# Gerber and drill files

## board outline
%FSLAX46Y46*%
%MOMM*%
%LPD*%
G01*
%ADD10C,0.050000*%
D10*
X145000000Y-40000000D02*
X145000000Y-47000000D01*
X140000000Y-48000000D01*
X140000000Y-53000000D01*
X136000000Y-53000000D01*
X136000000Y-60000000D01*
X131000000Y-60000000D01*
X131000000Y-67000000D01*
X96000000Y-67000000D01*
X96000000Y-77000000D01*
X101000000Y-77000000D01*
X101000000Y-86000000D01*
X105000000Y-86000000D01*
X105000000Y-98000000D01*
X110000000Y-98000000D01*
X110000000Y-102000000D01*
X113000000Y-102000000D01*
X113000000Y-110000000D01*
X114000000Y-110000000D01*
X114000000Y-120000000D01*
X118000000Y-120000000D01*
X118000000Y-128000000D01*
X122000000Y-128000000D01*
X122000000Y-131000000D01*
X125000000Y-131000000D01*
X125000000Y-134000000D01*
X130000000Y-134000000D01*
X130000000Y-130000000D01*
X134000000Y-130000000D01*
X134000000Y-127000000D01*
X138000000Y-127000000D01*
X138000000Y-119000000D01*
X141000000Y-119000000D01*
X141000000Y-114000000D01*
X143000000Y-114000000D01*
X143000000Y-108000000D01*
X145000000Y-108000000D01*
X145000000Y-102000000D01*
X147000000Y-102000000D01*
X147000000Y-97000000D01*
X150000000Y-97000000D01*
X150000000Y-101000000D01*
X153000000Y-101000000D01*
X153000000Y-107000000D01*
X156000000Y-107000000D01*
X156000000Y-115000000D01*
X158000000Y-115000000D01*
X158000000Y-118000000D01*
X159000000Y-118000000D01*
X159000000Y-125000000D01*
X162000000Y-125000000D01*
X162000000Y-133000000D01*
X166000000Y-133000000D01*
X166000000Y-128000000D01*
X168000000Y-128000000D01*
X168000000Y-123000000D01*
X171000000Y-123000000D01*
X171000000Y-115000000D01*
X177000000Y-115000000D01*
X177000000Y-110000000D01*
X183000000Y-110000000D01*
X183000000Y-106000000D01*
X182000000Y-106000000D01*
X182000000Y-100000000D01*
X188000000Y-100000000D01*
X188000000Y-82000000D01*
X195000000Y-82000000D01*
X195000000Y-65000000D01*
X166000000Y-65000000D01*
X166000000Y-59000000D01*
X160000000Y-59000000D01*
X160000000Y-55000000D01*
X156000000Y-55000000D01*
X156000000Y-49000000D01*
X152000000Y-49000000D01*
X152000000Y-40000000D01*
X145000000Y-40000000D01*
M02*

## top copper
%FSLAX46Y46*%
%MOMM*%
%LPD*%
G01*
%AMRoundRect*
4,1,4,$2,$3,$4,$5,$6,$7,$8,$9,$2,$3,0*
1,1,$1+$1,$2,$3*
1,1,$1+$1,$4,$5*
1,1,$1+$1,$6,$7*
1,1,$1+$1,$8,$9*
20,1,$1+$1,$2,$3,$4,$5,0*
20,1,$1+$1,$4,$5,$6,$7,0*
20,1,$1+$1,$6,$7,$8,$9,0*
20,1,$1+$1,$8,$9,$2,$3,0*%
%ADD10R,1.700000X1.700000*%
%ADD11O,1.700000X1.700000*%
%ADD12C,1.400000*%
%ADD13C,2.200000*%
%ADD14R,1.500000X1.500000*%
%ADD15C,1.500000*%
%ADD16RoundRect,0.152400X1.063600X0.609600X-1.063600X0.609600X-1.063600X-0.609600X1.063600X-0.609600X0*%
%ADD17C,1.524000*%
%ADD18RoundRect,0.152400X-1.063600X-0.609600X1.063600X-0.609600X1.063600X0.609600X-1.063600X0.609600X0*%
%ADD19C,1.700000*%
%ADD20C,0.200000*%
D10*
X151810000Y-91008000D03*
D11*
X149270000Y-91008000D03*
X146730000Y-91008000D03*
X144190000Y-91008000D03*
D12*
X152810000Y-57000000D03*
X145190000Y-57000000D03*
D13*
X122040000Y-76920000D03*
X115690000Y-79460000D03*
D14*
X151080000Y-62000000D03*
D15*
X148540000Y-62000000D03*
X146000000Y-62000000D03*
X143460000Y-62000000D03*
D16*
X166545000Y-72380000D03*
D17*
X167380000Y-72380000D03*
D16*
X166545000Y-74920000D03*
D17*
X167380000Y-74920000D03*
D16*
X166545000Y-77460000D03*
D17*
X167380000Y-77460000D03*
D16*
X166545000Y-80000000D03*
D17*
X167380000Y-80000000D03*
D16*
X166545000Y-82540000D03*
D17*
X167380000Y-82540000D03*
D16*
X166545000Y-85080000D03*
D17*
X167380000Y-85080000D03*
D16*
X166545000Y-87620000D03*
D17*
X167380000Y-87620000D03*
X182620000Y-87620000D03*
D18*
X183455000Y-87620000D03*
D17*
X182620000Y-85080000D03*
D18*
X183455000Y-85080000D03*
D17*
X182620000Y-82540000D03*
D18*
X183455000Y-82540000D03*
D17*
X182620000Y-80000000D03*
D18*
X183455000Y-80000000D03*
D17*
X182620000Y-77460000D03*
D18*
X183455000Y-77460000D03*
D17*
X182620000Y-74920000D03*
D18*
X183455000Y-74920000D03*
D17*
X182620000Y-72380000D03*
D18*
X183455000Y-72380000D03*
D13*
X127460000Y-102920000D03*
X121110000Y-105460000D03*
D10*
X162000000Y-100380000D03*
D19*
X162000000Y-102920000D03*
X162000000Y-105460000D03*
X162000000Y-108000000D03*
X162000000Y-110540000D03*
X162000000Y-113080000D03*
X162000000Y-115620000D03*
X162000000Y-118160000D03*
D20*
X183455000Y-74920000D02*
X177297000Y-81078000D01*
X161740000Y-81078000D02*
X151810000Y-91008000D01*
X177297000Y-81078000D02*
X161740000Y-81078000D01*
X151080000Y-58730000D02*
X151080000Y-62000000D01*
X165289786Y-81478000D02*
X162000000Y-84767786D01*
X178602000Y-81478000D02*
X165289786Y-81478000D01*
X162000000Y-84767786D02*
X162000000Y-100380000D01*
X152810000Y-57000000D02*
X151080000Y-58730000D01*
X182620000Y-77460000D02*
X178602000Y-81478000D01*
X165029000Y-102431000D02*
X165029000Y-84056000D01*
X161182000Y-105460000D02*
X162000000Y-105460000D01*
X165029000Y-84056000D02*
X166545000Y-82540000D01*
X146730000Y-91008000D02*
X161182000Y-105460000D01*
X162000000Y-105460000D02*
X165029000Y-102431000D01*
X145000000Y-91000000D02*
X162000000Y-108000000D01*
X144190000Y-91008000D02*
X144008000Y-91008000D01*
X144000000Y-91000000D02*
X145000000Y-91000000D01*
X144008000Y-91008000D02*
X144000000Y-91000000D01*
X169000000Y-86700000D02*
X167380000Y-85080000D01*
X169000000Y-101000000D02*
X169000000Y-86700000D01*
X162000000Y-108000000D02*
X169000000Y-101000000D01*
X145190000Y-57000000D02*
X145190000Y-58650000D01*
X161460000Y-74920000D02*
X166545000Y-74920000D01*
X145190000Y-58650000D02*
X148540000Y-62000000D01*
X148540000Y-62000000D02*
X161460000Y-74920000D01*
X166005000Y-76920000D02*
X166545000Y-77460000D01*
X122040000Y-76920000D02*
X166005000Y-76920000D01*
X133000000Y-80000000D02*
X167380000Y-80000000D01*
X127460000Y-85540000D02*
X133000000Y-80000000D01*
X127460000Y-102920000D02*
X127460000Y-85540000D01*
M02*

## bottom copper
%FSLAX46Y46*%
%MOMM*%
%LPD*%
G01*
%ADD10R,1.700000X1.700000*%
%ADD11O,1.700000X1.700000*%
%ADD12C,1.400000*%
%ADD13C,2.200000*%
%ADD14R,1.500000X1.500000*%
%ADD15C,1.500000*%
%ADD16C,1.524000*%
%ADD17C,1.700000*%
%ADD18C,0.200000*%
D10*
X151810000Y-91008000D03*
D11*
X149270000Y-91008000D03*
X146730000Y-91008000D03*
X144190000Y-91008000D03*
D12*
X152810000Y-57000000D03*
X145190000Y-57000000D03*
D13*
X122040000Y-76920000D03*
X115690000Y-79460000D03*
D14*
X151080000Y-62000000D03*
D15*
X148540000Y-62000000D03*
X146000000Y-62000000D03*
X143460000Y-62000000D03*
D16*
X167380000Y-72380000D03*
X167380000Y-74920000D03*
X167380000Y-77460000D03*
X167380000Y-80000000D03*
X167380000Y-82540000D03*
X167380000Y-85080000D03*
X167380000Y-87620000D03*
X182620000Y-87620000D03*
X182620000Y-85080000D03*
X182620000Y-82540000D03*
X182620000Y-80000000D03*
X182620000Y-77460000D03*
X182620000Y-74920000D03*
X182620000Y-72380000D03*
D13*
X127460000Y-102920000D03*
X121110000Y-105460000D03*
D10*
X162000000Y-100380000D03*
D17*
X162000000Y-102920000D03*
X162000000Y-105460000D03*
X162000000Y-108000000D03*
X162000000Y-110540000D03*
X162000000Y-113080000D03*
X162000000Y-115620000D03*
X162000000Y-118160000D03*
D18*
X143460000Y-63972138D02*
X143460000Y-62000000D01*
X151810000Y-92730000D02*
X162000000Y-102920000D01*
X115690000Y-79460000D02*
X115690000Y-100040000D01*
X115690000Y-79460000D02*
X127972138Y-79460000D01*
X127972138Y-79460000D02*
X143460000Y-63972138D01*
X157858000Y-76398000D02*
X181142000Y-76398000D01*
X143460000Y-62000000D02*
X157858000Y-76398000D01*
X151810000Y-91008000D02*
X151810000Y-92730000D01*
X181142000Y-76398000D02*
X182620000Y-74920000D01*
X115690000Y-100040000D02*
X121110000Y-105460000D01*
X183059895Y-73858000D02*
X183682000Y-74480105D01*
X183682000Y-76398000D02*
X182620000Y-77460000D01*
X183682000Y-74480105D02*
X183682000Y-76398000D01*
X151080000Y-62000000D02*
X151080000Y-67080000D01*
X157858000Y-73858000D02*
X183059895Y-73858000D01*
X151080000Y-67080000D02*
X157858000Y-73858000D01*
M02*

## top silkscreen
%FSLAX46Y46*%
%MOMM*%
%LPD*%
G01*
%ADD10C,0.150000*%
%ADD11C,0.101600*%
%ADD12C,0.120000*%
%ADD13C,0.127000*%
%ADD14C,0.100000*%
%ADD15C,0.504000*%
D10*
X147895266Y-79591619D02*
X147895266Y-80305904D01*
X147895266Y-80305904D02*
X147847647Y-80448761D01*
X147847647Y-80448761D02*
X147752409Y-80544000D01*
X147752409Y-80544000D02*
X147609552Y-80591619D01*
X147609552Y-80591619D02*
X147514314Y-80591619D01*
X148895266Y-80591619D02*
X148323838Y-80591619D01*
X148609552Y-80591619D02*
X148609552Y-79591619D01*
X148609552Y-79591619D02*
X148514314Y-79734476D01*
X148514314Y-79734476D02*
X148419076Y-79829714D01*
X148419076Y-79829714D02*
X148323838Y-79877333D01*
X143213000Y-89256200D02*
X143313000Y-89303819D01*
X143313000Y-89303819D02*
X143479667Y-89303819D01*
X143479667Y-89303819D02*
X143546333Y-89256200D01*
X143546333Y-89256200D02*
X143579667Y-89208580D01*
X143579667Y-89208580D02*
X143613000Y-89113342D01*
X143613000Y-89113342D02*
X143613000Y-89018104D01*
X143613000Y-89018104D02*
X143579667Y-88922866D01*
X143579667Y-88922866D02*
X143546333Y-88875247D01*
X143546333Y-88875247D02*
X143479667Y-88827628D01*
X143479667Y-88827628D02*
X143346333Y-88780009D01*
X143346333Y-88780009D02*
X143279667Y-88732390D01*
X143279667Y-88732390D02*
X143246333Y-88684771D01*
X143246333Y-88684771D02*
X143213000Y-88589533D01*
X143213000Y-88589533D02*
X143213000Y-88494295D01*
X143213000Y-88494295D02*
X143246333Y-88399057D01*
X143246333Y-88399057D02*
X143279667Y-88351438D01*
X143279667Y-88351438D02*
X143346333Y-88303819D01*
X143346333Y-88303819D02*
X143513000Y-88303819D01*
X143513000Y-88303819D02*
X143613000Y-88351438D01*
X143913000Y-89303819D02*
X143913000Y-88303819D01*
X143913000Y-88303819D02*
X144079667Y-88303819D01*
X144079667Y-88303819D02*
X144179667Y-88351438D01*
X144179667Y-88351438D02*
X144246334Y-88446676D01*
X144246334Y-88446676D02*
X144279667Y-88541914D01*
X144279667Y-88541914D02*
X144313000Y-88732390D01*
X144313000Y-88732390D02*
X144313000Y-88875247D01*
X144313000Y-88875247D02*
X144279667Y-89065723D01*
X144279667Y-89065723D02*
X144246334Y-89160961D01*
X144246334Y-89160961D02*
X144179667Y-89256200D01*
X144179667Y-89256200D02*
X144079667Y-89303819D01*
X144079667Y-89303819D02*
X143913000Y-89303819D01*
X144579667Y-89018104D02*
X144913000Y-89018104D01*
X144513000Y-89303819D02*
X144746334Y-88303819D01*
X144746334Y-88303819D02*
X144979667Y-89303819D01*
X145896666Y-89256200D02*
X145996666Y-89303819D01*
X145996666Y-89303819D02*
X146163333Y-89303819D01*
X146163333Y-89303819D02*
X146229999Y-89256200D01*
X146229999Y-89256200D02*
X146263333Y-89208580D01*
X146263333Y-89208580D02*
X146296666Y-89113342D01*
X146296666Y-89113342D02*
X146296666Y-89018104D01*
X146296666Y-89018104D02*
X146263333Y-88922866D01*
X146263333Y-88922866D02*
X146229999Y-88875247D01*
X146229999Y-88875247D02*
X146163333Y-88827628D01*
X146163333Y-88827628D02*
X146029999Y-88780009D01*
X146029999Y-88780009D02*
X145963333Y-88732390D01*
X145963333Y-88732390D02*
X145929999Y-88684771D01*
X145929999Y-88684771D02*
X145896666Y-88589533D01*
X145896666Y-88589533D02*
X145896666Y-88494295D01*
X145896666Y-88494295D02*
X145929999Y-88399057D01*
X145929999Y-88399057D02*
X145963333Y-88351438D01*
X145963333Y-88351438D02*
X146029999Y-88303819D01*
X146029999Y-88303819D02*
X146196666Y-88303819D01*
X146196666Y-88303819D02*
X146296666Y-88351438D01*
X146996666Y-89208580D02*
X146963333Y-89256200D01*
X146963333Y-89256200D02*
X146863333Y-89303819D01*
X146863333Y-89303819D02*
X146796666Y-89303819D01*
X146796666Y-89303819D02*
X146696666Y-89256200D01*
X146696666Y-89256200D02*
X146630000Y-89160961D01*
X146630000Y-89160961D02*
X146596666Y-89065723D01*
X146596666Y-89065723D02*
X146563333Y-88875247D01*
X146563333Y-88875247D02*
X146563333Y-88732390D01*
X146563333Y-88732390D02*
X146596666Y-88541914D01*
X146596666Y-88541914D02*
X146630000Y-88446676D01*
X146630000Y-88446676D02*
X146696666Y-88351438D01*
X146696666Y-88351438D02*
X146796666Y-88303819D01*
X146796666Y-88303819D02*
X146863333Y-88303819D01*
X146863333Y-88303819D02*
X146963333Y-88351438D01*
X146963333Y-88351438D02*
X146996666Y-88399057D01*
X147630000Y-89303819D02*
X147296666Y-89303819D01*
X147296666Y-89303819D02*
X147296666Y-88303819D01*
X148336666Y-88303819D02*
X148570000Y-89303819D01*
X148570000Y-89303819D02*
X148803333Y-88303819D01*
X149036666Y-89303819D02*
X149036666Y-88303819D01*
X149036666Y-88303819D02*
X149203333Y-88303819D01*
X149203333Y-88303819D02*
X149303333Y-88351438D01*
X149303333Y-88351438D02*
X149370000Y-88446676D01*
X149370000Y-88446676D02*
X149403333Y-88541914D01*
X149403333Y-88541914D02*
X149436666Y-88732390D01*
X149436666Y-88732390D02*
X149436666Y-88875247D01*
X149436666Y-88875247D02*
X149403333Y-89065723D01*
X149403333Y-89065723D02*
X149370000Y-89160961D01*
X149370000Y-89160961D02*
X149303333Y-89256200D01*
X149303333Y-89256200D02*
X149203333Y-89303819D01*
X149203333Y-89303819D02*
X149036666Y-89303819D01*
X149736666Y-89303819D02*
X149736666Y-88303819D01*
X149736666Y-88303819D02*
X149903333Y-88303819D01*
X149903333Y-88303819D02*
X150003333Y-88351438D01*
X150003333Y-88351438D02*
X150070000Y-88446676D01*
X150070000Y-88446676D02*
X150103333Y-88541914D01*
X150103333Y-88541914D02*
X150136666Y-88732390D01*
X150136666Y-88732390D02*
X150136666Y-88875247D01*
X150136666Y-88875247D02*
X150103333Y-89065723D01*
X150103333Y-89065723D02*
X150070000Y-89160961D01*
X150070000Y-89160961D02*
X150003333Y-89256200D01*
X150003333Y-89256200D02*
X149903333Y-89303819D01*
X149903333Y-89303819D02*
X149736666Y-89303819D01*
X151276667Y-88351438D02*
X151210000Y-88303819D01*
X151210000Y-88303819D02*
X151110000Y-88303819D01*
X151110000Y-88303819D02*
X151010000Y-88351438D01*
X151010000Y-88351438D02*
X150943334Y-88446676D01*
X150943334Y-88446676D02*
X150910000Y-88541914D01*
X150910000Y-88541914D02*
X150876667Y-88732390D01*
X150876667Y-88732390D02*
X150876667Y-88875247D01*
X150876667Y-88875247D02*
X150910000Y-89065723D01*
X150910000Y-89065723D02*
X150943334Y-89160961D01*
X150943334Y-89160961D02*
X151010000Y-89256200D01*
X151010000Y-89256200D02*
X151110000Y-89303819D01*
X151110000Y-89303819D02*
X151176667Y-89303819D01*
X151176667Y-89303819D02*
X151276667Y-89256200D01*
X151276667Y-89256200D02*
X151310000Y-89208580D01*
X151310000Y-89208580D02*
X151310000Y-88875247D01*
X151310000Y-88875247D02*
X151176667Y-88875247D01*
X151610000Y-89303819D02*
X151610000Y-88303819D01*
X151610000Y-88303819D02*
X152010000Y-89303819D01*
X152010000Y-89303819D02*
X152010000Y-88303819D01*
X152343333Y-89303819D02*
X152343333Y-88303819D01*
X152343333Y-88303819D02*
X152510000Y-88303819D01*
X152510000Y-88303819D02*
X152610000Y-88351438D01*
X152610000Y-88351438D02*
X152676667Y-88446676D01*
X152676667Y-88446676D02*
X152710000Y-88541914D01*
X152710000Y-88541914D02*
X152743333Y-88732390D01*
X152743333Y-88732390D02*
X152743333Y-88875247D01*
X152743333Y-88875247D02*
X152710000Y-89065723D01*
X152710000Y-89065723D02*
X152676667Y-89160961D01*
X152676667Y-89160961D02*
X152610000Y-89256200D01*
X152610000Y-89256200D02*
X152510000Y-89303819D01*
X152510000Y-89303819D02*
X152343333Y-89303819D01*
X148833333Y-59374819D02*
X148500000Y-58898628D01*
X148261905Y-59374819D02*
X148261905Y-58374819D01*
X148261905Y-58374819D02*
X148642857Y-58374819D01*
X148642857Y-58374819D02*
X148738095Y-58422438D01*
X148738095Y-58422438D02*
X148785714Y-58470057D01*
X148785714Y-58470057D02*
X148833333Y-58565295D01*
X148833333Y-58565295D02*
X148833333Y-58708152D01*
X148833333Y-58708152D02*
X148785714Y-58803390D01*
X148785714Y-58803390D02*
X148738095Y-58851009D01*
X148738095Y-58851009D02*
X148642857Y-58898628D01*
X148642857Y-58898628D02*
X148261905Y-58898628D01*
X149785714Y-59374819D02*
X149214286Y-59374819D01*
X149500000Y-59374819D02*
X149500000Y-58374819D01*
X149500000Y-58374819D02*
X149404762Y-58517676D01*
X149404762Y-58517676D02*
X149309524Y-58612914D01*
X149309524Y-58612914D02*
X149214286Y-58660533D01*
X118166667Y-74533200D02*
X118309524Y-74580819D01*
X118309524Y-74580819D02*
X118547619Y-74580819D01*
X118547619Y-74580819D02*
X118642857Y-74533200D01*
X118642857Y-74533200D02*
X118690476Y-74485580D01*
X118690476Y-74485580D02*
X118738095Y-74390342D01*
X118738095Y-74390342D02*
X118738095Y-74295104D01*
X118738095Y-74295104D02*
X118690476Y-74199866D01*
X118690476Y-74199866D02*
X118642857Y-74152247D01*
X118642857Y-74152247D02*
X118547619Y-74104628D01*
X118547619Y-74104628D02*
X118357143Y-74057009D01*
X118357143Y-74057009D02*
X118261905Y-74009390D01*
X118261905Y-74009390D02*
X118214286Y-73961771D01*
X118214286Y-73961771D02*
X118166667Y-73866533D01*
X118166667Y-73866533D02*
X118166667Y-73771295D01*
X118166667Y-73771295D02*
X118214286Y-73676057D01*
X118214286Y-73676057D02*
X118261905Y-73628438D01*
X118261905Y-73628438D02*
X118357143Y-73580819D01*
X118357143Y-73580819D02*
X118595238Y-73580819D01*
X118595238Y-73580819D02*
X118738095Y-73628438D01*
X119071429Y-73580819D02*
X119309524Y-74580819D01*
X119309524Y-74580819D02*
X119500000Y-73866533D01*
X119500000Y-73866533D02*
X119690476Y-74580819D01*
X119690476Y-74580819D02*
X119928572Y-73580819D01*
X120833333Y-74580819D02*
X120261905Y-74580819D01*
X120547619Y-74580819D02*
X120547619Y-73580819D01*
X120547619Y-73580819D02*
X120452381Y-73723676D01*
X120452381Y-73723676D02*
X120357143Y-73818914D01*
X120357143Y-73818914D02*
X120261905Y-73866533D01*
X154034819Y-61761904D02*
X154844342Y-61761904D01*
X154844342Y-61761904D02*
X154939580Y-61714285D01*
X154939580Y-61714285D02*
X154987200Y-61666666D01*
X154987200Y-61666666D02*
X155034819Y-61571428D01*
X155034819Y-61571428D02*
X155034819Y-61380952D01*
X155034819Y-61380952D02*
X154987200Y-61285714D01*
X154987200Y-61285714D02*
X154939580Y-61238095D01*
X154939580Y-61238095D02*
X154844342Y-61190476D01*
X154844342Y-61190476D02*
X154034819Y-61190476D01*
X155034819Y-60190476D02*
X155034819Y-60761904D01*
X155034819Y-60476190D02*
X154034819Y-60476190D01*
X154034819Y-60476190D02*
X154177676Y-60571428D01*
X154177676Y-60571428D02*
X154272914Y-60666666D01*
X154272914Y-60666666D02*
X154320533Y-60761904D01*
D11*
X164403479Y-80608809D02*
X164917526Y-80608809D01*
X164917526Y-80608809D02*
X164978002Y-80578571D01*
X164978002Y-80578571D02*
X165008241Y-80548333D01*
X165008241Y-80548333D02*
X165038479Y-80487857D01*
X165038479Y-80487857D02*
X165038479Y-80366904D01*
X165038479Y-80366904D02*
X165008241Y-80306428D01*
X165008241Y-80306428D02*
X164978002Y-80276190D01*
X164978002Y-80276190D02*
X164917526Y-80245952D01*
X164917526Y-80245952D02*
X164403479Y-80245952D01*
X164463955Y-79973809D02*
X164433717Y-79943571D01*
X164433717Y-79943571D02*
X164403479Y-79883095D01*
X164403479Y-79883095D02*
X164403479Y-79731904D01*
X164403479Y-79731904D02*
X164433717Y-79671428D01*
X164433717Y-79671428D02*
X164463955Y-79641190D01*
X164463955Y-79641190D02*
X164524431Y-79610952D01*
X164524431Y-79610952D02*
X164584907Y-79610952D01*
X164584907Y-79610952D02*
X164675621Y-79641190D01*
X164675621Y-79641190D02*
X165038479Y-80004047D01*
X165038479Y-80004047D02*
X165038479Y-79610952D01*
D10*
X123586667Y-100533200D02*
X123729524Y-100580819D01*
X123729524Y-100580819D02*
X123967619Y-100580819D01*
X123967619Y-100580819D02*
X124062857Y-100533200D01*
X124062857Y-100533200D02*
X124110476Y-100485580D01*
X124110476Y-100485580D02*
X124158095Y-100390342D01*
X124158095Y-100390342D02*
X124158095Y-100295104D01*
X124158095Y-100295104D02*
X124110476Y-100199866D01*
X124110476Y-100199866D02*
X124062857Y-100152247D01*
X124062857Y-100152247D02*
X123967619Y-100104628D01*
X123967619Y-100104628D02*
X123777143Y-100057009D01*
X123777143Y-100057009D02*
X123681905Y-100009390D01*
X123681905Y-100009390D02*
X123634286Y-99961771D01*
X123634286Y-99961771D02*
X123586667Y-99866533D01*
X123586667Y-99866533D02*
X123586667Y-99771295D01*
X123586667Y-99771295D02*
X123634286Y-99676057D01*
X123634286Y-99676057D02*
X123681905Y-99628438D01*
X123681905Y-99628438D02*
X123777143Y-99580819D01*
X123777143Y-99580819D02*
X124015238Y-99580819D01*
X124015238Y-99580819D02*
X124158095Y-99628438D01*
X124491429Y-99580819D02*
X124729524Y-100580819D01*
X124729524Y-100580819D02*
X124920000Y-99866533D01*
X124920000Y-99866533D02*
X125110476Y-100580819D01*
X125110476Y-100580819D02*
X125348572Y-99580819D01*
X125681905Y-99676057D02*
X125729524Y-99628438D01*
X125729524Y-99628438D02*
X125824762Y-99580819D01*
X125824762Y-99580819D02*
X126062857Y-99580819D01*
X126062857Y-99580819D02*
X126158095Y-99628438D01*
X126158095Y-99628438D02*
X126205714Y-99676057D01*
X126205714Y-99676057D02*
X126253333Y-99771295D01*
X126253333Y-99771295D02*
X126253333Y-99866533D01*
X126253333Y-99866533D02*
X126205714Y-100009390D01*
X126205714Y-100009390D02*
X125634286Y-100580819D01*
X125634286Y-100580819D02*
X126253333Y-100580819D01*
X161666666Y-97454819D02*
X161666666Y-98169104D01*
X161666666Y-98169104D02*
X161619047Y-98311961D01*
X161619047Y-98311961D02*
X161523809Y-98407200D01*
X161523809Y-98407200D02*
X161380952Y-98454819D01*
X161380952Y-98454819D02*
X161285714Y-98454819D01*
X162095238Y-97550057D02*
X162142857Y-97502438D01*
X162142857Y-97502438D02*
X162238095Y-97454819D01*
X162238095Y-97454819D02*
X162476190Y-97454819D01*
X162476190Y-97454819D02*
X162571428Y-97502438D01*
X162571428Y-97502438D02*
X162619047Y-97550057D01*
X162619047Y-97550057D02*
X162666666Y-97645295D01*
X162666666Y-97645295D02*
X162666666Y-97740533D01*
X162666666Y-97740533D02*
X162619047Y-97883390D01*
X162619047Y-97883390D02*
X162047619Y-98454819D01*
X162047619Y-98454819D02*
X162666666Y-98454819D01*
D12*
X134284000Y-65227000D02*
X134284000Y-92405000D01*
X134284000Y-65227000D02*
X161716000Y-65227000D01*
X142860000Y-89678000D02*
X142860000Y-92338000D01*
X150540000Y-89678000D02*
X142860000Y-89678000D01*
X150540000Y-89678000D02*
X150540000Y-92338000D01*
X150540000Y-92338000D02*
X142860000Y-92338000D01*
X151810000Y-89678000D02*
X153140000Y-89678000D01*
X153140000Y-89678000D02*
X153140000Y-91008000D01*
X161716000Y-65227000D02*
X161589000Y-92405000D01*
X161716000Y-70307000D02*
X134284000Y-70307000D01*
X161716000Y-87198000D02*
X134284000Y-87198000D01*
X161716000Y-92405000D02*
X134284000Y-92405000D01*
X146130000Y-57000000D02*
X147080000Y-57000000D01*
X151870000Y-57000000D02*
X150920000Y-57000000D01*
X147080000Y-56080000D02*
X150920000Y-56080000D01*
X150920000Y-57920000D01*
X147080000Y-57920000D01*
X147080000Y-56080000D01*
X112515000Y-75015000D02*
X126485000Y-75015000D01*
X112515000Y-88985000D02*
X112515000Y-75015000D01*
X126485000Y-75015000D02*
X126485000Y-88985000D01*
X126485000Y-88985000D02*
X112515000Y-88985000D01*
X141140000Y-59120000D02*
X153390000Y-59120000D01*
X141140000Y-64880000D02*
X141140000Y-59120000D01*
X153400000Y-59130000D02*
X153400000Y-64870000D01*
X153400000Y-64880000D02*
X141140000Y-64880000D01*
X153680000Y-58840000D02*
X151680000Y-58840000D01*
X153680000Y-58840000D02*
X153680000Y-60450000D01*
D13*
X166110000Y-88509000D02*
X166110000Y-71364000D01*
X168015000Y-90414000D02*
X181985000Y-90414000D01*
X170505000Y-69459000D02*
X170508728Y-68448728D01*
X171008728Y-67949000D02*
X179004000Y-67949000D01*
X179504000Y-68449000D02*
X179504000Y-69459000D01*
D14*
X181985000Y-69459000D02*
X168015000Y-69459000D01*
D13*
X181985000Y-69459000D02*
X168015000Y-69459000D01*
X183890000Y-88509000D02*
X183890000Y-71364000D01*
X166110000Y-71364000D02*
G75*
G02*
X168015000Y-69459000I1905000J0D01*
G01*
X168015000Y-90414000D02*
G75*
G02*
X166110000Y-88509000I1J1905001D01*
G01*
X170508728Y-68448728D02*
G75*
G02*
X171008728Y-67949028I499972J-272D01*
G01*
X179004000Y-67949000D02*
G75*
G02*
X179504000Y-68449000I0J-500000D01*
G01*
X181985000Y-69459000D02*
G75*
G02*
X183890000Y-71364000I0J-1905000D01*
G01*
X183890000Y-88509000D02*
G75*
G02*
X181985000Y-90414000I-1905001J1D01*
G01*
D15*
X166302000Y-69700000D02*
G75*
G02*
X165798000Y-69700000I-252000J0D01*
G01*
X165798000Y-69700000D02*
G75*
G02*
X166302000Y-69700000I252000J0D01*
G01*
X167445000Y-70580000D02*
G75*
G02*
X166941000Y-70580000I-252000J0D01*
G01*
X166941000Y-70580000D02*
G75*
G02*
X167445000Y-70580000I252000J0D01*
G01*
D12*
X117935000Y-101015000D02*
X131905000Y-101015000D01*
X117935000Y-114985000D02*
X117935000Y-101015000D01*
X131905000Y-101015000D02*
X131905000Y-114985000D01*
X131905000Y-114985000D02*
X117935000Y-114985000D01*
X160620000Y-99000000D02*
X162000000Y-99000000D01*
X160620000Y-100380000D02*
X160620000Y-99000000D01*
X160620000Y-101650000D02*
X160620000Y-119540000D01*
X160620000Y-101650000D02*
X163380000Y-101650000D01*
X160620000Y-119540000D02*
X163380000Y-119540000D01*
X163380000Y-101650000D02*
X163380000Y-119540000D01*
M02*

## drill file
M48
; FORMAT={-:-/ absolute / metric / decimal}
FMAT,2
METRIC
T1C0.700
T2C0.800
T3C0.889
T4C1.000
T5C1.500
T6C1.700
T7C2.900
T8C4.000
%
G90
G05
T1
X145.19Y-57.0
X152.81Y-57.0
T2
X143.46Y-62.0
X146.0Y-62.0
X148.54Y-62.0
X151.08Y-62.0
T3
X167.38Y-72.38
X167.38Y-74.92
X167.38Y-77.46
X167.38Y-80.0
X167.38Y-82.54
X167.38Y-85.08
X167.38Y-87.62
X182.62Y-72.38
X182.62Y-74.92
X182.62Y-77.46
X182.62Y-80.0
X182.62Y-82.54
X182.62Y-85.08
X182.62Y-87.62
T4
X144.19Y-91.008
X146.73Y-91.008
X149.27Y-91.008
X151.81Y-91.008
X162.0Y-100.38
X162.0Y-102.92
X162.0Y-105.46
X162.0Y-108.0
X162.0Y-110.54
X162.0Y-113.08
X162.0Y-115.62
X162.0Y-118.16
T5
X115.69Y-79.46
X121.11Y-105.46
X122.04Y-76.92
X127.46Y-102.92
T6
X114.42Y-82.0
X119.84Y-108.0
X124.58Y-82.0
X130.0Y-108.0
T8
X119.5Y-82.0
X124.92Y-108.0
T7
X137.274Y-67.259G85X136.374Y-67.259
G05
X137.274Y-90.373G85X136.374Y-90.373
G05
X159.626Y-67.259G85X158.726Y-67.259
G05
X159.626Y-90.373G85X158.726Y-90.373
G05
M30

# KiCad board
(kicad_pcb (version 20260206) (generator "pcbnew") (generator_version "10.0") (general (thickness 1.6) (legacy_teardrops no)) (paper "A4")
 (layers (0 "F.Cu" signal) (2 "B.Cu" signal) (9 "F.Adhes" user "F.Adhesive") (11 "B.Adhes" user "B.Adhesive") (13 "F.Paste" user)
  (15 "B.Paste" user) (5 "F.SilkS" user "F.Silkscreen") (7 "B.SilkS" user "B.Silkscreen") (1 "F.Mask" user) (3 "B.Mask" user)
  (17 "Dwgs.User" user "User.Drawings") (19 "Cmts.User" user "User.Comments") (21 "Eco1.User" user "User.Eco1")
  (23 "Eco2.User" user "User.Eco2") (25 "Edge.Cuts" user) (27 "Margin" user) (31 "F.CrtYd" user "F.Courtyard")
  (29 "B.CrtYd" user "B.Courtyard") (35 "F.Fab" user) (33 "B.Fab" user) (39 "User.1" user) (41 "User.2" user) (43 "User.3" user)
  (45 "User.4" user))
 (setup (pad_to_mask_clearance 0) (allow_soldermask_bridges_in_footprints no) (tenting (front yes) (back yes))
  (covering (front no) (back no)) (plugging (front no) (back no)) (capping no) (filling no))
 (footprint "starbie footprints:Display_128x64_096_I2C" (layer "F.Cu") (at 148 91.008 180)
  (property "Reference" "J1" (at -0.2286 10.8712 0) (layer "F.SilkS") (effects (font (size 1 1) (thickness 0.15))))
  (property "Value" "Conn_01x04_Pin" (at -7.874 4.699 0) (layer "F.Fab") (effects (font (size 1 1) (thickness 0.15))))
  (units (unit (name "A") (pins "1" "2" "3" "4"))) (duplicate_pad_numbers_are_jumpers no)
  (fp_line (start 13.716 25.781) (end 13.716 -1.397) (stroke (width 0.12) (type solid)) (layer "F.SilkS"))
  (fp_line (start 13.716 25.781) (end -13.716 25.781) (stroke (width 0.12) (type solid)) (layer "F.SilkS"))
  (fp_line (start 5.14 1.33) (end 5.14 -1.33) (stroke (width 0.12) (type solid)) (layer "F.SilkS"))
  (fp_line (start -2.54 1.33) (end 5.14 1.33) (stroke (width 0.12) (type solid)) (layer "F.SilkS"))
  (fp_line (start -2.54 1.33) (end -2.54 -1.33) (stroke (width 0.12) (type solid)) (layer "F.SilkS"))
  (fp_line (start -2.54 -1.33) (end 5.14 -1.33) (stroke (width 0.12) (type solid)) (layer "F.SilkS"))
  (fp_line (start -3.81 1.33) (end -5.14 1.33) (stroke (width 0.12) (type solid)) (layer "F.SilkS"))
  (fp_line (start -5.14 1.33) (end -5.14 0) (stroke (width 0.12) (type solid)) (layer "F.SilkS"))
  (fp_line (start -13.716 25.781) (end -13.589 -1.397) (stroke (width 0.12) (type solid)) (layer "F.SilkS"))
  (fp_line (start -13.716 20.701) (end 13.716 20.701) (stroke (width 0.12) (type solid)) (layer "F.SilkS"))
  (fp_line (start -13.716 3.81) (end 13.716 3.81) (stroke (width 0.12) (type solid)) (layer "F.SilkS"))
  (fp_line (start -13.716 -1.397) (end 13.716 -1.397) (stroke (width 0.12) (type solid)) (layer "F.SilkS"))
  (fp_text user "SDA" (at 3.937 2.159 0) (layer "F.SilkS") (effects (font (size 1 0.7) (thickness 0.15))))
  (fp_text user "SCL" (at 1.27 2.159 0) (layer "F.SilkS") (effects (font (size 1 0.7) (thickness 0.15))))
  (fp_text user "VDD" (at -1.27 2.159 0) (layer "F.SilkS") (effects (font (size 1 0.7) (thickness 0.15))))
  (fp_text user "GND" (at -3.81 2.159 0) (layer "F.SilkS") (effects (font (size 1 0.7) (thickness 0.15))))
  (pad "" np_thru_hole oval (at -11.176 0.635 180) (size 3.8 2.9) (drill oval 3.8 2.9) (layers "*.Cu" "*.Mask"))
  (pad "" np_thru_hole oval (at -11.176 23.749 180) (size 3.8 2.9) (drill oval 3.8 2.9) (layers "*.Cu" "*.Mask"))
  (pad "" np_thru_hole oval (at 11.176 0.635 180) (size 3.8 2.9) (drill oval 3.8 2.9) (layers "*.Cu" "*.Mask"))
  (pad "" np_thru_hole oval (at 11.176 23.749 180) (size 3.8 2.9) (drill oval 3.8 2.9) (layers "*.Cu" "*.Mask"))
  (pad "1" thru_hole rect (at -3.81 0 270) (size 1.7 1.7) (drill 1) (layers "*.Cu" "*.Mask") (remove_unused_layers no) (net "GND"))
  (pad "2" thru_hole oval (at -1.27 0 270) (size 1.7 1.7) (drill 1) (layers "*.Cu" "*.Mask") (remove_unused_layers no) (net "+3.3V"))
  (pad "3" thru_hole oval (at 1.27 0 270) (size 1.7 1.7) (drill 1) (layers "*.Cu" "*.Mask") (remove_unused_layers no) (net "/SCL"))
  (pad "4" thru_hole oval (at 3.81 0 270) (size 1.7 1.7) (drill 1) (layers "*.Cu" "*.Mask") (remove_unused_layers no) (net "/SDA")))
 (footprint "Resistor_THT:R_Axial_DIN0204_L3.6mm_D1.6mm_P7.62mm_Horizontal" (layer "F.Cu") (at 152.81 57 180)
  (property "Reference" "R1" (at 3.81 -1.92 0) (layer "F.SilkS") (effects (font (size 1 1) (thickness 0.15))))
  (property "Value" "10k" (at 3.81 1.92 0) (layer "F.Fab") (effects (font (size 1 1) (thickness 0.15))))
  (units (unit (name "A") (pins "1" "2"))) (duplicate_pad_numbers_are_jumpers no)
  (fp_line (start 6.68 0) (end 5.73 0) (stroke (width 0.12) (type solid)) (layer "F.SilkS"))
  (fp_line (start 0.94 0) (end 1.89 0) (stroke (width 0.12) (type solid)) (layer "F.SilkS"))
  (fp_rect (start 1.89 -0.92) (end 5.73 0.92) (stroke (width 0.12) (type solid)) (fill no) (layer "F.SilkS"))
  (pad "1" thru_hole circle (at 0 0 180) (size 1.4 1.4) (drill 0.7) (layers "*.Cu" "*.Mask") (remove_unused_layers no) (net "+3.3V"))
  (pad "2" thru_hole circle (at 7.62 0 180) (size 1.4 1.4) (drill 0.7) (layers "*.Cu" "*.Mask") (remove_unused_layers no)
   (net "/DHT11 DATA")))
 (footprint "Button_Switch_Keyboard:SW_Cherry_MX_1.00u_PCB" (layer "F.Cu") (at 122.04 76.92)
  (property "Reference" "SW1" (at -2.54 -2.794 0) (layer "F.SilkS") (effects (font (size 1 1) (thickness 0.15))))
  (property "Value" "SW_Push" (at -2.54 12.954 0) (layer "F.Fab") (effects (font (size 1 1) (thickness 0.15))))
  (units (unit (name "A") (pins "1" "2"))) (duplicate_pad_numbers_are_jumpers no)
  (fp_line (start -9.525 -1.905) (end 4.445 -1.905) (stroke (width 0.12) (type solid)) (layer "F.SilkS"))
  (fp_line (start -9.525 12.065) (end -9.525 -1.905) (stroke (width 0.12) (type solid)) (layer "F.SilkS"))
  (fp_line (start 4.445 -1.905) (end 4.445 12.065) (stroke (width 0.12) (type solid)) (layer "F.SilkS"))
  (fp_line (start 4.445 12.065) (end -9.525 12.065) (stroke (width 0.12) (type solid)) (layer "F.SilkS"))
  (pad "" np_thru_hole circle (at -7.62 5.08) (size 1.7 1.7) (drill 1.7) (layers "*.Cu" "*.Mask"))
  (pad "" np_thru_hole circle (at -2.54 5.08) (size 4 4) (drill 4) (layers "*.Cu" "*.Mask"))
  (pad "" np_thru_hole circle (at 2.54 5.08) (size 1.7 1.7) (drill 1.7) (layers "*.Cu" "*.Mask"))
  (pad "1" thru_hole circle (at 0 0) (size 2.2 2.2) (drill 1.5) (layers "*.Cu" "*.Mask") (remove_unused_layers no) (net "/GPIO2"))
  (pad "2" thru_hole circle (at -6.35 2.54) (size 2.2 2.2) (drill 1.5) (layers "*.Cu" "*.Mask") (remove_unused_layers no) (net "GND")))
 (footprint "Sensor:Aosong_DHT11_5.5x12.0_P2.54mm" (layer "F.Cu") (at 151.08 62 -90)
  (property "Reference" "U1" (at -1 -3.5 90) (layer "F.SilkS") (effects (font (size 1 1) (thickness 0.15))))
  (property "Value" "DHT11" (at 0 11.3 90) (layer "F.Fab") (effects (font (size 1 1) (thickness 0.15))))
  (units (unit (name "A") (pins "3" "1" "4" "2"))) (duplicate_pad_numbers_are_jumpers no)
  (fp_line (start -2.88 9.94) (end -2.88 -2.31) (stroke (width 0.12) (type solid)) (layer "F.SilkS"))
  (fp_line (start 2.88 9.94) (end -2.88 9.94) (stroke (width 0.12) (type solid)) (layer "F.SilkS"))
  (fp_line (start -2.87 -2.32) (end 2.87 -2.32) (stroke (width 0.12) (type solid)) (layer "F.SilkS"))
  (fp_line (start 2.88 -2.32) (end 2.88 9.94) (stroke (width 0.12) (type solid)) (layer "F.SilkS"))
  (fp_line (start -3.16 -2.6) (end -3.16 -0.6) (stroke (width 0.12) (type solid)) (layer "F.SilkS"))
  (fp_line (start -3.16 -2.6) (end -1.55 -2.6) (stroke (width 0.12) (type solid)) (layer "F.SilkS"))
  (pad "1" thru_hole rect (at 0 0 270) (size 1.5 1.5) (drill 0.8) (layers "*.Cu" "*.Mask") (remove_unused_layers no) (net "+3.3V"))
  (pad "2" thru_hole circle (at 0 2.54 270) (size 1.5 1.5) (drill 0.8) (layers "*.Cu" "*.Mask") (remove_unused_layers no)
   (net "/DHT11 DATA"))
  (pad "3" thru_hole circle (at 0 5.08 270) (size 1.5 1.5) (drill 0.8) (layers "*.Cu" "*.Mask") (remove_unused_layers no)
   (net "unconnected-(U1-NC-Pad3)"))
  (pad "4" thru_hole circle (at 0 7.62 270) (size 1.5 1.5) (drill 0.8) (layers "*.Cu" "*.Mask") (remove_unused_layers no) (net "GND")))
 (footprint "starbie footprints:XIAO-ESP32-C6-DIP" (layer "F.Cu") (at 175 80 90)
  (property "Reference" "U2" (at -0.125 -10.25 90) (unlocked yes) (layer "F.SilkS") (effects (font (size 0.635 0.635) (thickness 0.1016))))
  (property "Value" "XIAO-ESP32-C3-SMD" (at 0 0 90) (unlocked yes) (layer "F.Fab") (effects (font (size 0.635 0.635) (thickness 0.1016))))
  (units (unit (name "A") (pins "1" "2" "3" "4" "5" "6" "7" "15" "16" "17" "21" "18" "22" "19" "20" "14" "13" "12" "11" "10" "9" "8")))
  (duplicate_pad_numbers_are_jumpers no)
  (fp_line (start -8.509 -8.89) (end 8.636 -8.89) (stroke (width 0.127) (type solid)) (layer "F.SilkS"))
  (fp_line (start -10.414 -6.985) (end -10.414 6.985) (stroke (width 0.127) (type solid)) (layer "F.SilkS"))
  (fp_line (start 10.541 -4.495) (end 11.551272 -4.491272) (stroke (width 0.127) (type solid)) (layer "F.SilkS"))
  (fp_line (start 12.051 -3.991272) (end 12.051 4.004) (stroke (width 0.127) (type solid)) (layer "F.SilkS"))
  (fp_line (start 11.551 4.504) (end 10.541 4.504) (stroke (width 0.127) (type solid)) (layer "F.SilkS"))
  (fp_line (start 10.541 6.985) (end 10.541 -6.985) (stroke (width 0.1) (type solid)) (layer "F.SilkS"))
  (fp_line (start 10.541 6.985) (end 10.541 -6.985) (stroke (width 0.127) (type solid)) (layer "F.SilkS"))
  (fp_line (start -8.509 8.89) (end 8.636 8.89) (stroke (width 0.127) (type solid)) (layer "F.SilkS"))
  (fp_arc (start 8.636 -8.89) (mid 9.983038 -8.332038) (end 10.541 -6.985) (stroke (width 0.127) (type solid)) (layer "F.SilkS"))
  (fp_arc (start -10.414 -6.985) (mid -9.856038 -8.332038) (end -8.509 -8.89) (stroke (width 0.127) (type solid)) (layer "F.SilkS"))
  (fp_arc (start 11.551272 -4.491272) (mid 11.904644 -4.344724) (end 12.051 -3.991272) (stroke (width 0.127) (type default))
   (layer "F.SilkS"))
  (fp_arc (start 12.051 4.004) (mid 11.904553 4.357553) (end 11.551 4.504) (stroke (width 0.127) (type default)) (layer "F.SilkS"))
  (fp_arc (start 10.541 6.985) (mid 9.983038 8.332038) (end 8.636 8.89) (stroke (width 0.127) (type solid)) (layer "F.SilkS"))
  (fp_arc (start -8.509 8.89) (mid -9.856038 8.332038) (end -10.414 6.985) (stroke (width 0.127) (type solid)) (layer "F.SilkS"))
  (fp_circle (center 10.3 -8.95) (end 10.554 -8.95) (stroke (width 0.5) (type solid)) (fill yes) (layer "F.SilkS"))
  (fp_circle (center 9.42 -7.807) (end 9.674 -7.807) (stroke (width 0.5) (type solid)) (fill yes) (layer "F.SilkS"))
  (pad "1" smd roundrect (at 7.62 -8.455 180) (size 2.432 1.524) (layers "F.Cu" "F.Mask") (roundrect_rratio 0.1)
   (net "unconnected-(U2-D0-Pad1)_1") (thermal_bridge_angle 45))
  (pad "1" thru_hole circle (at 7.62 -7.62 180) (size 1.524 1.524) (drill 0.889) (layers "*.Cu" "*.Mask") (remove_unused_layers no)
   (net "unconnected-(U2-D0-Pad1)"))
  (pad "2" smd roundrect (at 5.08 -8.455 180) (size 2.432 1.524) (layers "F.Cu" "F.Mask") (roundrect_rratio 0.1) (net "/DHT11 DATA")
   (thermal_bridge_angle 45))
  (pad "2" thru_hole circle (at 5.08 -7.62 180) (size 1.524 1.524) (drill 0.889) (layers "*.Cu" "*.Mask") (remove_unused_layers no)
   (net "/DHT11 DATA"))
  (pad "3" smd roundrect (at 2.54 -8.455 180) (size 2.432 1.524) (layers "F.Cu" "F.Mask") (roundrect_rratio 0.1) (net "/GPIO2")
   (thermal_bridge_angle 45))
  (pad "3" thru_hole circle (at 2.54 -7.62 180) (size 1.524 1.524) (drill 0.889) (layers "*.Cu" "*.Mask") (remove_unused_layers no)
   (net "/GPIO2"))
  (pad "4" smd roundrect (at 0 -8.455 180) (size 2.432 1.524) (layers "F.Cu" "F.Mask") (roundrect_rratio 0.1) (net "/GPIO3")
   (thermal_bridge_angle 45))
  (pad "4" thru_hole circle (at 0 -7.62 180) (size 1.524 1.524) (drill 0.889) (layers "*.Cu" "*.Mask") (remove_unused_layers no)
   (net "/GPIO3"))
  (pad "5" smd roundrect (at -2.54 -8.455 180) (size 2.432 1.524) (layers "F.Cu" "F.Mask") (roundrect_rratio 0.1) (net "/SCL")
   (thermal_bridge_angle 45))
  (pad "5" thru_hole circle (at -2.54 -7.62 180) (size 1.524 1.524) (drill 0.889) (layers "*.Cu" "*.Mask") (remove_unused_layers no)
   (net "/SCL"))
  (pad "6" smd roundrect (at -5.08 -8.455 180) (size 2.432 1.524) (layers "F.Cu" "F.Mask") (roundrect_rratio 0.1) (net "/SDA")
   (thermal_bridge_angle 45))
  (pad "6" thru_hole circle (at -5.08 -7.62 180) (size 1.524 1.524) (drill 0.889) (layers "*.Cu" "*.Mask") (remove_unused_layers no)
   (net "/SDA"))
  (pad "7" smd roundrect (at -7.62 -8.455 180) (size 2.432 1.524) (layers "F.Cu" "F.Mask") (roundrect_rratio 0.1)
   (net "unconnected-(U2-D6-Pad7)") (thermal_bridge_angle 45))
  (pad "7" thru_hole circle (at -7.62 -7.62 180) (size 1.524 1.524) (drill 0.889) (layers "*.Cu" "*.Mask") (remove_unused_layers no)
   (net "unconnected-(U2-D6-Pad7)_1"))
  (pad "8" thru_hole circle (at -7.62 7.62) (size 1.524 1.524) (drill 0.889) (layers "*.Cu" "*.Mask") (remove_unused_layers no)
   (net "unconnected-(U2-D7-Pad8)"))
  (pad "8" smd roundrect (at -7.62 8.455) (size 2.432 1.524) (layers "F.Cu" "F.Mask") (roundrect_rratio 0.1)
   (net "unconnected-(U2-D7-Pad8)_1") (thermal_bridge_angle 45))
  (pad "9" thru_hole circle (at -5.08 7.62) (size 1.524 1.524) (drill 0.889) (layers "*.Cu" "*.Mask") (remove_unused_layers no)
   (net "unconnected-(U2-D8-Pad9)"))
  (pad "9" smd roundrect (at -5.08 8.455) (size 2.432 1.524) (layers "F.Cu" "F.Mask") (roundrect_rratio 0.1)
   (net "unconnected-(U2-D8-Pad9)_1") (thermal_bridge_angle 45))
  (pad "10" thru_hole circle (at -2.54 7.62) (size 1.524 1.524) (drill 0.889) (layers "*.Cu" "*.Mask") (remove_unused_layers no)
   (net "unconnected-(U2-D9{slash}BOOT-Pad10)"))
  (pad "10" smd roundrect (at -2.54 8.455) (size 2.432 1.524) (layers "F.Cu" "F.Mask") (roundrect_rratio 0.1)
   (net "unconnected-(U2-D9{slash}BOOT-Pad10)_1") (thermal_bridge_angle 45))
  (pad "11" thru_hole circle (at 0 7.62) (size 1.524 1.524) (drill 0.889) (layers "*.Cu" "*.Mask") (remove_unused_layers no)
   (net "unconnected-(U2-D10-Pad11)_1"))
  (pad "11" smd roundrect (at 0 8.455) (size 2.432 1.524) (layers "F.Cu" "F.Mask") (roundrect_rratio 0.1) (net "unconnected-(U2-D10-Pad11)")
   (thermal_bridge_angle 45))
  (pad "12" thru_hole circle (at 2.54 7.62) (size 1.524 1.524) (drill 0.889) (layers "*.Cu" "*.Mask") (remove_unused_layers no)
   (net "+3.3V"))
  (pad "12" smd roundrect (at 2.54 8.455) (size 2.432 1.524) (layers "F.Cu" "F.Mask") (roundrect_rratio 0.1) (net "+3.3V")
   (thermal_bridge_angle 45))
  (pad "13" thru_hole circle (at 5.08 7.62) (size 1.524 1.524) (drill 0.889) (layers "*.Cu" "*.Mask") (remove_unused_layers no) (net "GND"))
  (pad "13" smd roundrect (at 5.08 8.455) (size 2.432 1.524) (layers "F.Cu" "F.Mask") (roundrect_rratio 0.1) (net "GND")
   (thermal_bridge_angle 45))
  (pad "14" thru_hole circle (at 7.62 7.62) (size 1.524 1.524) (drill 0.889) (layers "*.Cu" "*.Mask") (remove_unused_layers no) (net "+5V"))
  (pad "14" smd roundrect (at 7.62 8.455) (size 2.432 1.524) (layers "F.Cu" "F.Mask") (roundrect_rratio 0.1) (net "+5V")
   (thermal_bridge_angle 45)))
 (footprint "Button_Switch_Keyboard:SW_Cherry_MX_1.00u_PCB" (layer "F.Cu") (at 127.46 102.92)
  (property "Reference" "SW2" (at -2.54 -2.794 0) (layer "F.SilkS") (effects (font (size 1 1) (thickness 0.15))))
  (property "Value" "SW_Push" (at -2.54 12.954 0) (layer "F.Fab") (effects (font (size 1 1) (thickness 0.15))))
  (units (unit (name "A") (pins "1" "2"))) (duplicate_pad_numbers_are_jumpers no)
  (fp_line (start -9.525 -1.905) (end 4.445 -1.905) (stroke (width 0.12) (type solid)) (layer "F.SilkS"))
  (fp_line (start -9.525 12.065) (end -9.525 -1.905) (stroke (width 0.12) (type solid)) (layer "F.SilkS"))
  (fp_line (start 4.445 -1.905) (end 4.445 12.065) (stroke (width 0.12) (type solid)) (layer "F.SilkS"))
  (fp_line (start 4.445 12.065) (end -9.525 12.065) (stroke (width 0.12) (type solid)) (layer "F.SilkS"))
  (pad "" np_thru_hole circle (at -7.62 5.08) (size 1.7 1.7) (drill 1.7) (layers "*.Cu" "*.Mask"))
  (pad "" np_thru_hole circle (at -2.54 5.08) (size 4 4) (drill 4) (layers "*.Cu" "*.Mask"))
  (pad "" np_thru_hole circle (at 2.54 5.08) (size 1.7 1.7) (drill 1.7) (layers "*.Cu" "*.Mask"))
  (pad "1" thru_hole circle (at 0 0) (size 2.2 2.2) (drill 1.5) (layers "*.Cu" "*.Mask") (remove_unused_layers no) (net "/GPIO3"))
  (pad "2" thru_hole circle (at -6.35 2.54) (size 2.2 2.2) (drill 1.5) (layers "*.Cu" "*.Mask") (remove_unused_layers no) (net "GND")))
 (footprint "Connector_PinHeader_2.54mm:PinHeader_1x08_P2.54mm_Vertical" (layer "F.Cu") (at 162 100.38)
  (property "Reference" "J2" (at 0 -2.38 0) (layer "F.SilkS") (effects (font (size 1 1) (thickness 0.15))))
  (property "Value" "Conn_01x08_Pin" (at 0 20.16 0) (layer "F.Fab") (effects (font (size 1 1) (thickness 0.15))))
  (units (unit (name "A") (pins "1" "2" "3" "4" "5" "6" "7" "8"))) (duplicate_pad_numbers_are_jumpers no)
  (fp_line (start -1.38 -1.38) (end 0 -1.38) (stroke (width 0.12) (type solid)) (layer "F.SilkS"))
  (fp_line (start -1.38 0) (end -1.38 -1.38) (stroke (width 0.12) (type solid)) (layer "F.SilkS"))
  (fp_line (start -1.38 1.27) (end -1.38 19.16) (stroke (width 0.12) (type solid)) (layer "F.SilkS"))
  (fp_line (start -1.38 1.27) (end 1.38 1.27) (stroke (width 0.12) (type solid)) (layer "F.SilkS"))
  (fp_line (start -1.38 19.16) (end 1.38 19.16) (stroke (width 0.12) (type solid)) (layer "F.SilkS"))
  (fp_line (start 1.38 1.27) (end 1.38 19.16) (stroke (width 0.12) (type solid)) (layer "F.SilkS"))
  (pad "1" thru_hole rect (at 0 0) (size 1.7 1.7) (drill 1) (layers "*.Cu" "*.Mask") (remove_unused_layers no) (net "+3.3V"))
  (pad "2" thru_hole circle (at 0 2.54) (size 1.7 1.7) (drill 1) (layers "*.Cu" "*.Mask") (remove_unused_layers no) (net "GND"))
  (pad "3" thru_hole circle (at 0 5.08) (size 1.7 1.7) (drill 1) (layers "*.Cu" "*.Mask") (remove_unused_layers no) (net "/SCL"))
  (pad "4" thru_hole circle (at 0 7.62) (size 1.7 1.7) (drill 1) (layers "*.Cu" "*.Mask") (remove_unused_layers no) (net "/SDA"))
  (pad "5" thru_hole circle (at 0 10.16) (size 1.7 1.7) (drill 1) (layers "*.Cu" "*.Mask") (remove_unused_layers no)
   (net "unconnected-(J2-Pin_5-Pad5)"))
  (pad "6" thru_hole circle (at 0 12.7) (size 1.7 1.7) (drill 1) (layers "*.Cu" "*.Mask") (remove_unused_layers no)
   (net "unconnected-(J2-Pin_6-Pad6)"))
  (pad "7" thru_hole circle (at 0 15.24) (size 1.7 1.7) (drill 1) (layers "*.Cu" "*.Mask") (remove_unused_layers no)
   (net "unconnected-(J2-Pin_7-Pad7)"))
  (pad "8" thru_hole circle (at 0 17.78) (size 1.7 1.7) (drill 1) (layers "*.Cu" "*.Mask") (remove_unused_layers no)
   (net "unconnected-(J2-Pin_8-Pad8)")))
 (gr_poly
  (pts (xy 145 40) (xy 145 47) (xy 140 48) (xy 140 53) (xy 136 53) (xy 136 60) (xy 131 60) (xy 131 67) (xy 96 67) (xy 96 77) (xy 101 77)
   (xy 101 86) (xy 105 86) (xy 105 98) (xy 110 98) (xy 110 102) (xy 113 102) (xy 113 110) (xy 114 110) (xy 114 120) (xy 118 120)
   (xy 118 128) (xy 122 128) (xy 122 131) (xy 125 131) (xy 125 134) (xy 130 134) (xy 130 130) (xy 134 130) (xy 134 127) (xy 138 127)
   (xy 138 119) (xy 141 119) (xy 141 114) (xy 143 114) (xy 143 108) (xy 145 108) (xy 145 102) (xy 147 102) (xy 147 97) (xy 150 97)
   (xy 150 101) (xy 153 101) (xy 153 107) (xy 156 107) (xy 156 115) (xy 158 115) (xy 158 118) (xy 159 118) (xy 159 125) (xy 162 125)
   (xy 162 133) (xy 166 133) (xy 166 128) (xy 168 128) (xy 168 123) (xy 171 123) (xy 171 115) (xy 177 115) (xy 177 110) (xy 183 110)
   (xy 183 106) (xy 182 106) (xy 182 100) (xy 188 100) (xy 188 82) (xy 195 82) (xy 195 65) (xy 166 65) (xy 166 59) (xy 160 59) (xy 160 55)
   (xy 156 55) (xy 156 49) (xy 152 49) (xy 152 40))
  (stroke (width 0.05) (type solid)) (fill no) (layer "Edge.Cuts"))
 (segment (start 183.455 74.92) (end 177.297 81.078) (width 0.2) (layer "F.Cu") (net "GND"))
 (segment (start 161.74 81.078) (end 151.81 91.008) (width 0.2) (layer "F.Cu") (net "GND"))
 (segment (start 177.297 81.078) (end 161.74 81.078) (width 0.2) (layer "F.Cu") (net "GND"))
 (segment (start 143.46 63.972138) (end 143.46 62) (width 0.2) (layer "B.Cu") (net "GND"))
 (segment (start 151.81 92.73) (end 162 102.92) (width 0.2) (layer "B.Cu") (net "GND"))
 (segment (start 115.69 79.46) (end 115.69 100.04) (width 0.2) (layer "B.Cu") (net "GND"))
 (segment (start 115.69 79.46) (end 127.972138 79.46) (width 0.2) (layer "B.Cu") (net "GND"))
 (segment (start 127.972138 79.46) (end 143.46 63.972138) (width 0.2) (layer "B.Cu") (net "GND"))
 (segment (start 157.858 76.398) (end 181.142 76.398) (width 0.2) (layer "B.Cu") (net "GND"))
 (segment (start 143.46 62) (end 157.858 76.398) (width 0.2) (layer "B.Cu") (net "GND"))
 (segment (start 151.81 91.008) (end 151.81 92.73) (width 0.2) (layer "B.Cu") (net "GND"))
 (segment (start 181.142 76.398) (end 182.62 74.92) (width 0.2) (layer "B.Cu") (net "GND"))
 (segment (start 115.69 100.04) (end 121.11 105.46) (width 0.2) (layer "B.Cu") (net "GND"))
 (segment (start 151.08 58.73) (end 151.08 62) (width 0.2) (layer "F.Cu") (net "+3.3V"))
 (segment (start 165.289786 81.478) (end 162 84.767786) (width 0.2) (layer "F.Cu") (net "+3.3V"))
 (segment (start 178.602 81.478) (end 165.289786 81.478) (width 0.2) (layer "F.Cu") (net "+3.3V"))
 (segment (start 162 84.767786) (end 162 100.38) (width 0.2) (layer "F.Cu") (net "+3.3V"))
 (segment (start 152.81 57) (end 151.08 58.73) (width 0.2) (layer "F.Cu") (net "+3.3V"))
 (segment (start 182.62 77.46) (end 178.602 81.478) (width 0.2) (layer "F.Cu") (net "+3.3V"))
 (segment (start 183.059895 73.858) (end 183.682 74.480105) (width 0.2) (layer "B.Cu") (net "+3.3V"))
 (segment (start 183.682 76.398) (end 182.62 77.46) (width 0.2) (layer "B.Cu") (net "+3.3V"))
 (segment (start 183.682 74.480105) (end 183.682 76.398) (width 0.2) (layer "B.Cu") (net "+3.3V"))
 (segment (start 151.08 62) (end 151.08 67.08) (width 0.2) (layer "B.Cu") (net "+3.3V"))
 (segment (start 157.858 73.858) (end 183.059895 73.858) (width 0.2) (layer "B.Cu") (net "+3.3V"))
 (segment (start 151.08 67.08) (end 157.858 73.858) (width 0.2) (layer "B.Cu") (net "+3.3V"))
 (segment (start 165.029 102.431) (end 165.029 84.056) (width 0.2) (layer "F.Cu") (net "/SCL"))
 (segment (start 161.182 105.46) (end 162 105.46) (width 0.2) (layer "F.Cu") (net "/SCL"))
 (segment (start 165.029 84.056) (end 166.545 82.54) (width 0.2) (layer "F.Cu") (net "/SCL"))
 (segment (start 146.73 91.008) (end 161.182 105.46) (width 0.2) (layer "F.Cu") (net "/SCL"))
 (segment (start 162 105.46) (end 165.029 102.431) (width 0.2) (layer "F.Cu") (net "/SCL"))
 (segment (start 145 91) (end 162 108) (width 0.2) (layer "F.Cu") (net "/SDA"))
 (segment (start 144.19 91.008) (end 144.008 91.008) (width 0.2) (layer "F.Cu") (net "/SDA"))
 (segment (start 144 91) (end 145 91) (width 0.2) (layer "F.Cu") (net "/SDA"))
 (segment (start 144.008 91.008) (end 144 91) (width 0.2) (layer "F.Cu") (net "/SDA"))
 (segment (start 169 86.7) (end 167.38 85.08) (width 0.2) (layer "F.Cu") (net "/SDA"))
 (segment (start 169 101) (end 169 86.7) (width 0.2) (layer "F.Cu") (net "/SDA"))
 (segment (start 162 108) (end 169 101) (width 0.2) (layer "F.Cu") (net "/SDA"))
 (segment (start 145.19 57) (end 145.19 58.65) (width 0.2) (layer "F.Cu") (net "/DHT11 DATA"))
 (segment (start 161.46 74.92) (end 166.545 74.92) (width 0.2) (layer "F.Cu") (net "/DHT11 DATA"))
 (segment (start 145.19 58.65) (end 148.54 62) (width 0.2) (layer "F.Cu") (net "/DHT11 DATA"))
 (segment (start 148.54 62) (end 161.46 74.92) (width 0.2) (layer "F.Cu") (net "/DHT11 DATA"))
 (segment (start 166.005 76.92) (end 166.545 77.46) (width 0.2) (layer "F.Cu") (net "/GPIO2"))
 (segment (start 122.04 76.92) (end 166.005 76.92) (width 0.2) (layer "F.Cu") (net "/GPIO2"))
 (segment (start 133 80) (end 167.38 80) (width 0.2) (layer "F.Cu") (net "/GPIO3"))
 (segment (start 127.46 85.54) (end 133 80) (width 0.2) (layer "F.Cu") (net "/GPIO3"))
 (segment (start 127.46 102.92) (end 127.46 85.54) (width 0.2) (layer "F.Cu") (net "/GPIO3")))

